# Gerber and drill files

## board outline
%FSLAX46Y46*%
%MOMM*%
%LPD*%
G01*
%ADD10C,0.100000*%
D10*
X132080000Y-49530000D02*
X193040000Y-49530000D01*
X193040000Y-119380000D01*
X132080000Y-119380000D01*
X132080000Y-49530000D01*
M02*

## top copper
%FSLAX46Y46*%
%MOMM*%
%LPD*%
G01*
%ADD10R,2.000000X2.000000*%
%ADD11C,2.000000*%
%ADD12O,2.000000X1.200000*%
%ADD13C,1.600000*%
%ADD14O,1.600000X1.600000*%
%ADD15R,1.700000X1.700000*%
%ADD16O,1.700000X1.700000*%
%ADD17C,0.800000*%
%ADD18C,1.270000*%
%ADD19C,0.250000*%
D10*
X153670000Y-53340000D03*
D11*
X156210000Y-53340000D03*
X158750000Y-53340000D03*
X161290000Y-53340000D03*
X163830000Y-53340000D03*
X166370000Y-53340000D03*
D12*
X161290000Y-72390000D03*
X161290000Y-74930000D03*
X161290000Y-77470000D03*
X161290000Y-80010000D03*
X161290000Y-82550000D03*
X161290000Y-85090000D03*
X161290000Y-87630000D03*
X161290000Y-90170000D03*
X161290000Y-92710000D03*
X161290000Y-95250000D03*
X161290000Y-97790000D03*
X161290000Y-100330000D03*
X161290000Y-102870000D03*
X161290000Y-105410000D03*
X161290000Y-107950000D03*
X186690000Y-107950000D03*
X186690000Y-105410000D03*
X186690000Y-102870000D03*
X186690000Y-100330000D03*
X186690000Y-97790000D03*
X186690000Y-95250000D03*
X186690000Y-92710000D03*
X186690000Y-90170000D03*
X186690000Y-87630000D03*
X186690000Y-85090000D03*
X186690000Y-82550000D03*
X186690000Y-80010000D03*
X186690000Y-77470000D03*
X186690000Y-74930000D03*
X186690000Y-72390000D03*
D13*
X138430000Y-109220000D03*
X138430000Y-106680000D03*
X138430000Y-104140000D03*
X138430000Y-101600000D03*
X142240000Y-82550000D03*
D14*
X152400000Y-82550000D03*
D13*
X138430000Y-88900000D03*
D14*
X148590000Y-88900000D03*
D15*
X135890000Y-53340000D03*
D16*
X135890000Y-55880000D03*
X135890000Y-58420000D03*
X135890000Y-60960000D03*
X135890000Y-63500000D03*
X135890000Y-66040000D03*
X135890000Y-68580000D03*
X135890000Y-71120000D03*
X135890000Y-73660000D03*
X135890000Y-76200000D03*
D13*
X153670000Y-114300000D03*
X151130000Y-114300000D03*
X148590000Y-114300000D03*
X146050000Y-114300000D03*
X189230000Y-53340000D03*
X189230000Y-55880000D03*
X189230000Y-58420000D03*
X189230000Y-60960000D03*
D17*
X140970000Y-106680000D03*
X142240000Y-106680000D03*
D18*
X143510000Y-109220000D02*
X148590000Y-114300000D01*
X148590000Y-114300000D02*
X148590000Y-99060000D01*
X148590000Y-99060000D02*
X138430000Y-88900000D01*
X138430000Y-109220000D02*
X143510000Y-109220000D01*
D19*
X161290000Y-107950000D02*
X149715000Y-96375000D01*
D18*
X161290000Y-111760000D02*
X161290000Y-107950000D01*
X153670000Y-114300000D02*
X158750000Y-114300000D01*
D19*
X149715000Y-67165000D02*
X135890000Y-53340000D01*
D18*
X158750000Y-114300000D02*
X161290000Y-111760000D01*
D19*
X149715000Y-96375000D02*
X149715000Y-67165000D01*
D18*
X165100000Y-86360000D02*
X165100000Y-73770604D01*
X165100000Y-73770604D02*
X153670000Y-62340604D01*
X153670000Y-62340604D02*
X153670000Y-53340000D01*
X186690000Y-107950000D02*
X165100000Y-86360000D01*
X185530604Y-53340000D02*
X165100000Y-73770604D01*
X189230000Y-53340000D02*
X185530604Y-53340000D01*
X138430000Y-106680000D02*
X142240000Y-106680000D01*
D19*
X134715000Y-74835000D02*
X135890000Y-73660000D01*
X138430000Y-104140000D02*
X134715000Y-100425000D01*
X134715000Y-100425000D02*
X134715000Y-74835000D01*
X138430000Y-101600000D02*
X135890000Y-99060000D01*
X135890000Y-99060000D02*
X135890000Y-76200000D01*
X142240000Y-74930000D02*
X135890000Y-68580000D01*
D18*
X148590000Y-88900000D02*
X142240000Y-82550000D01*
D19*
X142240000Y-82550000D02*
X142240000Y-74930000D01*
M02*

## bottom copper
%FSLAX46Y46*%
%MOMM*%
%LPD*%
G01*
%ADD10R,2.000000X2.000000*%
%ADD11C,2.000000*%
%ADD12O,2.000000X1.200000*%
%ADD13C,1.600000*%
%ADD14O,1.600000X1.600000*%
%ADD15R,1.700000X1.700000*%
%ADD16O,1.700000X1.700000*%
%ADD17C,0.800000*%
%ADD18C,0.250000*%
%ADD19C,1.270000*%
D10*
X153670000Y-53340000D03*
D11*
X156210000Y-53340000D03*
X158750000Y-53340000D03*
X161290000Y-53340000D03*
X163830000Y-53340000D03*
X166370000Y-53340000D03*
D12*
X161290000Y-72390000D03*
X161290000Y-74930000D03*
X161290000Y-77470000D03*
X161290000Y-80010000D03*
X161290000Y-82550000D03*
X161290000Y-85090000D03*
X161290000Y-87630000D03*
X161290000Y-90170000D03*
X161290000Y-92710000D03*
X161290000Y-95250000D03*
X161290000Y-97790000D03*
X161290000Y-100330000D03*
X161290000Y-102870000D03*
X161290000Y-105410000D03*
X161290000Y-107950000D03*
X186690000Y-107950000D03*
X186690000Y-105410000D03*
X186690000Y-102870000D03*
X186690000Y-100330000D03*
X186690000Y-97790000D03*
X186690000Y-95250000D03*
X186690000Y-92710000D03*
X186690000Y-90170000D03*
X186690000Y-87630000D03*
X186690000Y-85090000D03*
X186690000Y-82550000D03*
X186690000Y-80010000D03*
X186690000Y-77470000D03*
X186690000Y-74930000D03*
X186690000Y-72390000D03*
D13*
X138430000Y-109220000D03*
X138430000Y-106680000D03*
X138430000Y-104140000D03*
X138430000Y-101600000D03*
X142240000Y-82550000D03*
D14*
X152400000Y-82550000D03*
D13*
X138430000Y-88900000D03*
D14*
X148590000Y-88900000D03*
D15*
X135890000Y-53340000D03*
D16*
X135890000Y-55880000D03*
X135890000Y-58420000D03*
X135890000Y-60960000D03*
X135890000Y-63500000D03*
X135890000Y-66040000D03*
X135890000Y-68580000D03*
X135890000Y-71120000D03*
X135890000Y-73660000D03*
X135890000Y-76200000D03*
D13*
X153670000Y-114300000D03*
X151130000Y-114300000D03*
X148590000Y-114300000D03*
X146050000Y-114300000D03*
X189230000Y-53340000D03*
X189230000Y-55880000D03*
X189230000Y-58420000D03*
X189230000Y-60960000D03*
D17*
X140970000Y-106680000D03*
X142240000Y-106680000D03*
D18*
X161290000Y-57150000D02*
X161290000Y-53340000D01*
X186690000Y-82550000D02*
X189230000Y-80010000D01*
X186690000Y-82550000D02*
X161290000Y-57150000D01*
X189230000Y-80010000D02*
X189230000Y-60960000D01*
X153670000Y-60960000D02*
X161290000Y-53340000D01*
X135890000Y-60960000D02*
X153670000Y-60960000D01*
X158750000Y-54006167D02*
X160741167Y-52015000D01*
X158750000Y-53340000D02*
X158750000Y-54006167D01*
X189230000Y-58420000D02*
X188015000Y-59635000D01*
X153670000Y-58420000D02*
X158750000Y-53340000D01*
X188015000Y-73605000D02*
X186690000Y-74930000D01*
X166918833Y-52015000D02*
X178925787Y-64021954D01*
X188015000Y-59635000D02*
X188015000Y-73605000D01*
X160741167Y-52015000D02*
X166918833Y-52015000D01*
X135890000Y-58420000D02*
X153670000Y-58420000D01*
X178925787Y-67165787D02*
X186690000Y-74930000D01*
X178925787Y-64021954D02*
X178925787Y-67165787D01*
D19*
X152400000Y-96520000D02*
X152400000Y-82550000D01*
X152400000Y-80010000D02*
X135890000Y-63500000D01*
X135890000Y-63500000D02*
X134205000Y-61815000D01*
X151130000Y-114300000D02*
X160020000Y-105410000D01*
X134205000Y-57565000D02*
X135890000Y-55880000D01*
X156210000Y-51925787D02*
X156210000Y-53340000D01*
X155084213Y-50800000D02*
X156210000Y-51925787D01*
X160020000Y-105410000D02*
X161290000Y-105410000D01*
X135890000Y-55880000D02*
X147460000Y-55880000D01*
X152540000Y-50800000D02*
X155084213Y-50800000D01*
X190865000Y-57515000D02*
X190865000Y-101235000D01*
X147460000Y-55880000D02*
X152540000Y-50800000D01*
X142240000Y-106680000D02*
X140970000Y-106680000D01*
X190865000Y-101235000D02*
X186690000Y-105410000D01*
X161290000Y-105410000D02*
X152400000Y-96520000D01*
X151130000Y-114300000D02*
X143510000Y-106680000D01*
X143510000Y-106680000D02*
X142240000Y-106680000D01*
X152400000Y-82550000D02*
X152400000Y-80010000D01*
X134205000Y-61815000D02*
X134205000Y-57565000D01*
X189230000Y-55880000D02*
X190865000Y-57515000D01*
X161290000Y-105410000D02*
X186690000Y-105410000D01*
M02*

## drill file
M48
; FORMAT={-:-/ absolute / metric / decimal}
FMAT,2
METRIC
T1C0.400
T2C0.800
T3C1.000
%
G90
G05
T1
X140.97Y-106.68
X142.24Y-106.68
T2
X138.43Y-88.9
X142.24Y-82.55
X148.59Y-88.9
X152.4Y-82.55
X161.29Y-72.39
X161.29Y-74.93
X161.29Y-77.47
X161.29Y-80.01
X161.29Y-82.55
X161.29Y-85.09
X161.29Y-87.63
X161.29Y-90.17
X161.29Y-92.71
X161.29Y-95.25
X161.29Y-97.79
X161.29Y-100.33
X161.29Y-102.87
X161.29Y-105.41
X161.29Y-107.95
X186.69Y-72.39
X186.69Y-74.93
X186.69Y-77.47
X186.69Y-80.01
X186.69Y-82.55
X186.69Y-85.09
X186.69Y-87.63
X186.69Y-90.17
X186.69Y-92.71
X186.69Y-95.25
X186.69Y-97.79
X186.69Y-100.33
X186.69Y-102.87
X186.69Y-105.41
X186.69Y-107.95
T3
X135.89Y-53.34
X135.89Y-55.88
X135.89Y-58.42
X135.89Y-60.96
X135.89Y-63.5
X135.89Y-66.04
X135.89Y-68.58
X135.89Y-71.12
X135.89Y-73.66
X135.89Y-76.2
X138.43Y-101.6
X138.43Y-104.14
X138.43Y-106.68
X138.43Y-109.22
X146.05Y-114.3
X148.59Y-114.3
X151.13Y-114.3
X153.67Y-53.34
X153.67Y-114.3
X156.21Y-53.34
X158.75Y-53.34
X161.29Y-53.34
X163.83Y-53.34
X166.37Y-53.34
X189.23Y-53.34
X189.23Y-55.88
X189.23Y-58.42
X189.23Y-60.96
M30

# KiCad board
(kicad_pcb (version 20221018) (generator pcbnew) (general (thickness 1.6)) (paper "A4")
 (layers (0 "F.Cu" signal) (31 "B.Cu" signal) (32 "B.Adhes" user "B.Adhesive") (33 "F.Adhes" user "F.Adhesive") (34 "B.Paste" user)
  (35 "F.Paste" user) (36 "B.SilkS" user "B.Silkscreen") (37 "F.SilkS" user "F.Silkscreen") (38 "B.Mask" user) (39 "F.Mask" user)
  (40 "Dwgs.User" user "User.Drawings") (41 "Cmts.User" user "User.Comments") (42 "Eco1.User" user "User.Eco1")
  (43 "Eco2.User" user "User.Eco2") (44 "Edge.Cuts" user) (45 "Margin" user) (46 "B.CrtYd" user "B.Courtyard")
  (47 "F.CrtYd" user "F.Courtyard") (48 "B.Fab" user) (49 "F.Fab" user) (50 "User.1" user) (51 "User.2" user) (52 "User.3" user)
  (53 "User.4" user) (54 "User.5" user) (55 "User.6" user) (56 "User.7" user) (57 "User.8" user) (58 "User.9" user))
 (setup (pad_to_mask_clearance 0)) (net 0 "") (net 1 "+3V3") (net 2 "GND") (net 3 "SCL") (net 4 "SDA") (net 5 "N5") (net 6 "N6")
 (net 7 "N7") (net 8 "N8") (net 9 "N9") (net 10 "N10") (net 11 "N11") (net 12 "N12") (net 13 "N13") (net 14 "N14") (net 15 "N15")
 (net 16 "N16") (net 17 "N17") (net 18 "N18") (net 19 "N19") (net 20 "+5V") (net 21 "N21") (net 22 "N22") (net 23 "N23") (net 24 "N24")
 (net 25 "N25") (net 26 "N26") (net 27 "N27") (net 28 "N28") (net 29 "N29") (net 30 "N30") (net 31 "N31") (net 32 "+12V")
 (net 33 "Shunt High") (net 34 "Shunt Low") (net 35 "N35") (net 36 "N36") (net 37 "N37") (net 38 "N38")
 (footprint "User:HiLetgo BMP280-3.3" (layer "F.Cu") (at 153.67 53.34 90)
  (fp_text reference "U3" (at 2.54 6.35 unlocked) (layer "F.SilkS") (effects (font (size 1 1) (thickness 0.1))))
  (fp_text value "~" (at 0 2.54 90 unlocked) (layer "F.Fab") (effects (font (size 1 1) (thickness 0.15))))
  (pad "1" thru_hole rect (at 0 0 90) (size 2 2) (drill 1) (layers "*.Cu" "*.Mask") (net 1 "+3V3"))
  (pad "2" thru_hole circle (at 0 2.54 90) (size 2 2) (drill 1) (layers "*.Cu" "*.Mask") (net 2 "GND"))
  (pad "3" thru_hole circle (at 0 5.08 90) (size 2 2) (drill 1) (layers "*.Cu" "*.Mask") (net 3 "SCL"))
  (pad "4" thru_hole circle (at 0 7.62 90) (size 2 2) (drill 1) (layers "*.Cu" "*.Mask") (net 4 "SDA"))
  (pad "5" thru_hole circle (at 0 10.16 90) (size 2 2) (drill 1) (layers "*.Cu" "*.Mask") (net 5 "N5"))
  (pad "6" thru_hole circle (at 0 12.7 90) (size 2 2) (drill 1) (layers "*.Cu" "*.Mask") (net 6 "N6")))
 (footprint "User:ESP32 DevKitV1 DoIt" (layer "F.Cu") (at 158.75 69.85)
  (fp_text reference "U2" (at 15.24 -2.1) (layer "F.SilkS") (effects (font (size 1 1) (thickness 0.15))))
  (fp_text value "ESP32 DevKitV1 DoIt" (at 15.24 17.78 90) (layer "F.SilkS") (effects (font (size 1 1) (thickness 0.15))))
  (pad "1" thru_hole oval (at 2.54 2.54 270) (size 1.2 2) (drill 0.8) (layers "*.Cu" "*.Mask") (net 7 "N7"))
  (pad "2" thru_hole oval (at 2.54 5.08 270) (size 1.2 2) (drill 0.8) (layers "*.Cu" "*.Mask") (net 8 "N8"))
  (pad "3" thru_hole oval (at 2.54 7.62 270) (size 1.2 2) (drill 0.8) (layers "*.Cu" "*.Mask") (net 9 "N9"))
  (pad "4" thru_hole oval (at 2.54 10.16 270) (size 1.2 2) (drill 0.8) (layers "*.Cu" "*.Mask") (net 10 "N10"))
  (pad "5" thru_hole oval (at 2.54 12.7 270) (size 1.2 2) (drill 0.8) (layers "*.Cu" "*.Mask") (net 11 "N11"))
  (pad "6" thru_hole oval (at 2.54 15.24 270) (size 1.2 2) (drill 0.8) (layers "*.Cu" "*.Mask") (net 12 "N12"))
  (pad "7" thru_hole oval (at 2.54 17.78 270) (size 1.2 2) (drill 0.8) (layers "*.Cu" "*.Mask") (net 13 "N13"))
  (pad "8" thru_hole oval (at 2.54 20.32 270) (size 1.2 2) (drill 0.8) (layers "*.Cu" "*.Mask") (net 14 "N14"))
  (pad "9" thru_hole oval (at 2.54 22.86 270) (size 1.2 2) (drill 0.8) (layers "*.Cu" "*.Mask") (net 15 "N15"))
  (pad "10" thru_hole oval (at 2.54 25.4 270) (size 1.2 2) (drill 0.8) (layers "*.Cu" "*.Mask") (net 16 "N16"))
  (pad "11" thru_hole oval (at 2.54 27.94 270) (size 1.2 2) (drill 0.8) (layers "*.Cu" "*.Mask") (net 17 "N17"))
  (pad "12" thru_hole oval (at 2.54 30.48 270) (size 1.2 2) (drill 0.8) (layers "*.Cu" "*.Mask") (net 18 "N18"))
  (pad "13" thru_hole oval (at 2.54 33.02 270) (size 1.2 2) (drill 0.8) (layers "*.Cu" "*.Mask") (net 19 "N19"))
  (pad "14" thru_hole oval (at 2.54 35.56 270) (size 1.2 2) (drill 0.8) (layers "*.Cu" "*.Mask") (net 2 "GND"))
  (pad "15" thru_hole oval (at 2.54 38.1 270) (size 1.2 2) (drill 0.8) (layers "*.Cu" "*.Mask") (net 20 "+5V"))
  (pad "16" thru_hole oval (at 27.94 38.1 270) (size 1.2 2) (drill 0.8) (layers "*.Cu" "*.Mask") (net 1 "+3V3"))
  (pad "17" thru_hole oval (at 27.94 35.56 270) (size 1.2 2) (drill 0.8) (layers "*.Cu" "*.Mask") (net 2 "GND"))
  (pad "18" thru_hole oval (at 27.94 33.02 270) (size 1.2 2) (drill 0.8) (layers "*.Cu" "*.Mask") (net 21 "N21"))
  (pad "19" thru_hole oval (at 27.94 30.48 270) (size 1.2 2) (drill 0.8) (layers "*.Cu" "*.Mask") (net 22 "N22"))
  (pad "20" thru_hole oval (at 27.94 27.94 270) (size 1.2 2) (drill 0.8) (layers "*.Cu" "*.Mask") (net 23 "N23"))
  (pad "21" thru_hole oval (at 27.94 25.4 270) (size 1.2 2) (drill 0.8) (layers "*.Cu" "*.Mask") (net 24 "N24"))
  (pad "22" thru_hole oval (at 27.94 22.86 270) (size 1.2 2) (drill 0.8) (layers "*.Cu" "*.Mask") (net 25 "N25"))
  (pad "23" thru_hole oval (at 27.94 20.32 270) (size 1.2 2) (drill 0.8) (layers "*.Cu" "*.Mask") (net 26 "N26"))
  (pad "24" thru_hole oval (at 27.94 17.78 270) (size 1.2 2) (drill 0.8) (layers "*.Cu" "*.Mask") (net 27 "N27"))
  (pad "25" thru_hole oval (at 27.94 15.24 270) (size 1.2 2) (drill 0.8) (layers "*.Cu" "*.Mask") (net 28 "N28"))
  (pad "26" thru_hole oval (at 27.94 12.7 270) (size 1.2 2) (drill 0.8) (layers "*.Cu" "*.Mask") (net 4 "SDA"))
  (pad "27" thru_hole oval (at 27.94 10.16 270) (size 1.2 2) (drill 0.8) (layers "*.Cu" "*.Mask") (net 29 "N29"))
  (pad "28" thru_hole oval (at 27.94 7.62 270) (size 1.2 2) (drill 0.8) (layers "*.Cu" "*.Mask") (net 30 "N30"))
  (pad "29" thru_hole oval (at 27.94 5.08 270) (size 1.2 2) (drill 0.8) (layers "*.Cu" "*.Mask") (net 3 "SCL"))
  (pad "30" thru_hole oval (at 27.94 2.54 270) (size 1.2 2) (drill 0.8) (layers "*.Cu" "*.Mask") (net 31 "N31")))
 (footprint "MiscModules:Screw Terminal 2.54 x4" (layer "F.Cu") (at 140.97 96.52 180)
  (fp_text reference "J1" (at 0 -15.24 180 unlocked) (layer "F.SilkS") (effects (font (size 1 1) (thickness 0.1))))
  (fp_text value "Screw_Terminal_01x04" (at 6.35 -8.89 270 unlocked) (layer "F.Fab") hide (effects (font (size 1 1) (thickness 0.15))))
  (pad "1" thru_hole circle (at 2.54 -12.7 90) (size 1.6 1.6) (drill 1) (layers "*.Cu" "*.Mask") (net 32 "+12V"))
  (pad "2" thru_hole circle (at 2.54 -10.16 90) (size 1.6 1.6) (drill 1) (layers "*.Cu" "*.Mask") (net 2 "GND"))
  (pad "3" thru_hole circle (at 2.54 -7.62 90) (size 1.6 1.6) (drill 1) (layers "*.Cu" "*.Mask") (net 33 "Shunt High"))
  (pad "4" thru_hole circle (at 2.54 -5.08 90) (size 1.6 1.6) (drill 1) (layers "*.Cu" "*.Mask") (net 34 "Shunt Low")))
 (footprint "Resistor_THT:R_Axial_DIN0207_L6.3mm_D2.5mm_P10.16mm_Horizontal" (layer "F.Cu") (at 142.24 82.55)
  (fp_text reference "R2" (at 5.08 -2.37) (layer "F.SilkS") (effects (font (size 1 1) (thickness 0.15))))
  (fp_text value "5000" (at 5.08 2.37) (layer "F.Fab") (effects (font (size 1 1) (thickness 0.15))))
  (pad "1" thru_hole circle (at 0 0) (size 1.6 1.6) (drill 0.8) (layers "*.Cu" "*.Mask") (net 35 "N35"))
  (pad "2" thru_hole oval (at 10.16 0) (size 1.6 1.6) (drill 0.8) (layers "*.Cu" "*.Mask") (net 2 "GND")))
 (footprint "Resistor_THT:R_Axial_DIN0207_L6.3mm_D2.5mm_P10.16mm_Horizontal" (layer "F.Cu") (at 138.43 88.9)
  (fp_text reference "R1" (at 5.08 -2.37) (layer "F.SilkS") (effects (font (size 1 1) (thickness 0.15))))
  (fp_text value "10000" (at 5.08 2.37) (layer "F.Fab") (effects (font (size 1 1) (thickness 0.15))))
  (pad "1" thru_hole circle (at 0 0) (size 1.6 1.6) (drill 0.8) (layers "*.Cu" "*.Mask") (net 32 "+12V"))
  (pad "2" thru_hole oval (at 10.16 0) (size 1.6 1.6) (drill 0.8) (layers "*.Cu" "*.Mask") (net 35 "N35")))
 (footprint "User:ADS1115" (layer "F.Cu") (at 135.89 53.34)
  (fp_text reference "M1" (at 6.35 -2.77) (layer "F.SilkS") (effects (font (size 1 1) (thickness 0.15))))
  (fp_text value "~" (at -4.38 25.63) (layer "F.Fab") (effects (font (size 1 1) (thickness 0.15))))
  (pad "1" thru_hole rect (at 0 0) (size 1.7 1.7) (drill 1) (layers "*.Cu" "*.Mask") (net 20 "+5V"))
  (pad "2" thru_hole oval (at 0 2.54) (size 1.7 1.7) (drill 1) (layers "*.Cu" "*.Mask") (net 2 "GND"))
  (pad "3" thru_hole oval (at 0 5.08) (size 1.7 1.7) (drill 1) (layers "*.Cu" "*.Mask") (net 3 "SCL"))
  (pad "4" thru_hole oval (at 0 7.62) (size 1.7 1.7) (drill 1) (layers "*.Cu" "*.Mask") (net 4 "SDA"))
  (pad "5" thru_hole oval (at 0 10.16) (size 1.7 1.7) (drill 1) (layers "*.Cu" "*.Mask") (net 2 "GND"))
  (pad "6" thru_hole oval (at 0 12.7) (size 1.7 1.7) (drill 1) (layers "*.Cu" "*.Mask") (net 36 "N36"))
  (pad "7" thru_hole oval (at 0 15.24) (size 1.7 1.7) (drill 1) (layers "*.Cu" "*.Mask") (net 35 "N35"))
  (pad "8" thru_hole oval (at 0 17.78) (size 1.7 1.7) (drill 1) (layers "*.Cu" "*.Mask") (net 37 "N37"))
  (pad "9" thru_hole oval (at 0 20.32) (size 1.7 1.7) (drill 1) (layers "*.Cu" "*.Mask") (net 33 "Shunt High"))
  (pad "10" thru_hole oval (at 0 22.86) (size 1.7 1.7) (drill 1) (layers "*.Cu" "*.Mask") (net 34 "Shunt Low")))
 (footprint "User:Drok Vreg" (layer "F.Cu") (at 149.86 111.76 -90)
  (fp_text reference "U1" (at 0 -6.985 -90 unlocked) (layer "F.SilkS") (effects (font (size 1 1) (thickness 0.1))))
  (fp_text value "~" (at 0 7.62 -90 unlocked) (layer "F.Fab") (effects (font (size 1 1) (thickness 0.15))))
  (pad "1" thru_hole circle (at 2.54 -3.81 180) (size 1.6 1.6) (drill 1) (layers "*.Cu" "*.Mask") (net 20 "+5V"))
  (pad "2" thru_hole circle (at 2.54 -1.27 180) (size 1.6 1.6) (drill 1) (layers "*.Cu" "*.Mask") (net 2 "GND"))
  (pad "3" thru_hole circle (at 2.54 1.27 180) (size 1.6 1.6) (drill 1) (layers "*.Cu" "*.Mask") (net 32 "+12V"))
  (pad "4" thru_hole circle (at 2.54 3.81 180) (size 1.6 1.6) (drill 1) (layers "*.Cu" "*.Mask") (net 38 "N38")))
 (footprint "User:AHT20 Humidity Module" (layer "F.Cu") (at 186.69 57.15)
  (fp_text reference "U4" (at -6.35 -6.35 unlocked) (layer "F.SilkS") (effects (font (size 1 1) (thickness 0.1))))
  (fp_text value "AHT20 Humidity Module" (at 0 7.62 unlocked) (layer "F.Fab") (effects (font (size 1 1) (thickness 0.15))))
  (pad "1" thru_hole circle (at 2.54 -3.81 270) (size 1.6 1.6) (drill 1) (layers "*.Cu" "*.Mask") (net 1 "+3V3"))
  (pad "2" thru_hole circle (at 2.54 -1.27 270) (size 1.6 1.6) (drill 1) (layers "*.Cu" "*.Mask") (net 2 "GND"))
  (pad "3" thru_hole circle (at 2.54 1.27 270) (size 1.6 1.6) (drill 1) (layers "*.Cu" "*.Mask") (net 3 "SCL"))
  (pad "4" thru_hole circle (at 2.54 3.81 270) (size 1.6 1.6) (drill 1) (layers "*.Cu" "*.Mask") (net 4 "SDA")))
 (gr_rect (start 132.08 49.53) (end 193.04 119.38) (stroke (width 0.1) (type default)) (fill none) (layer "Edge.Cuts"))
 (segment (start 143.51 109.22) (end 148.59 114.3) (width 1.27) (layer "F.Cu") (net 32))
 (segment (start 148.59 114.3) (end 148.59 99.06) (width 1.27) (layer "F.Cu") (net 32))
 (segment (start 148.59 99.06) (end 138.43 88.9) (width 1.27) (layer "F.Cu") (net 32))
 (segment (start 138.43 109.22) (end 143.51 109.22) (width 1.27) (layer "F.Cu") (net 32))
 (segment (start 161.29 107.95) (end 149.715 96.375) (width 0.25) (layer "F.Cu") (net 20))
 (segment (start 161.29 111.76) (end 161.29 107.95) (width 1.27) (layer "F.Cu") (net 20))
 (segment (start 153.67 114.3) (end 158.75 114.3) (width 1.27) (layer "F.Cu") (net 20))
 (segment (start 149.715 67.165) (end 135.89 53.34) (width 0.25) (layer "F.Cu") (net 20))
 (segment (start 158.75 114.3) (end 161.29 111.76) (width 1.27) (layer "F.Cu") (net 20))
 (segment (start 149.715 96.375) (end 149.715 67.165) (width 0.25) (layer "F.Cu") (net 20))
 (segment (start 165.1 86.36) (end 165.1 73.770604) (width 1.27) (layer "F.Cu") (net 1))
 (segment (start 165.1 73.770604) (end 153.67 62.340604) (width 1.27) (layer "F.Cu") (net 1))
 (segment (start 153.67 62.340604) (end 153.67 53.34) (width 1.27) (layer "F.Cu") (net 1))
 (segment (start 186.69 107.95) (end 165.1 86.36) (width 1.27) (layer "F.Cu") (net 1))
 (segment (start 185.530604 53.34) (end 165.1 73.770604) (width 1.27) (layer "F.Cu") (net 1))
 (segment (start 189.23 53.34) (end 185.530604 53.34) (width 1.27) (layer "F.Cu") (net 1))
 (segment (start 161.29 57.15) (end 161.29 53.34) (width 0.25) (layer "B.Cu") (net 4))
 (segment (start 186.69 82.55) (end 189.23 80.01) (width 0.25) (layer "B.Cu") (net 4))
 (segment (start 186.69 82.55) (end 161.29 57.15) (width 0.25) (layer "B.Cu") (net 4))
 (segment (start 189.23 80.01) (end 189.23 60.96) (width 0.25) (layer "B.Cu") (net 4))
 (segment (start 153.67 60.96) (end 161.29 53.34) (width 0.25) (layer "B.Cu") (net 4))
 (segment (start 135.89 60.96) (end 153.67 60.96) (width 0.25) (layer "B.Cu") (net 4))
 (segment (start 158.75 54.006167) (end 160.741167 52.015) (width 0.25) (layer "B.Cu") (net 3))
 (segment (start 158.75 53.34) (end 158.75 54.006167) (width 0.25) (layer "B.Cu") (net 3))
 (segment (start 189.23 58.42) (end 188.015 59.635) (width 0.25) (layer "B.Cu") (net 3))
 (segment (start 153.67 58.42) (end 158.75 53.34) (width 0.25) (layer "B.Cu") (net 3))
 (segment (start 188.015 73.605) (end 186.69 74.93) (width 0.25) (layer "B.Cu") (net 3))
 (segment (start 166.918833 52.015) (end 178.925787 64.021954) (width 0.25) (layer "B.Cu") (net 3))
 (segment (start 188.015 59.635) (end 188.015 73.605) (width 0.25) (layer "B.Cu") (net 3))
 (segment (start 160.741167 52.015) (end 166.918833 52.015) (width 0.25) (layer "B.Cu") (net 3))
 (segment (start 135.89 58.42) (end 153.67 58.42) (width 0.25) (layer "B.Cu") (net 3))
 (segment (start 178.925787 67.165787) (end 186.69 74.93) (width 0.25) (layer "B.Cu") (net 3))
 (segment (start 178.925787 64.021954) (end 178.925787 67.165787) (width 0.25) (layer "B.Cu") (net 3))
 (segment (start 138.43 106.68) (end 142.24 106.68) (width 1.27) (layer "F.Cu") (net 2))
 (via (at 140.97 106.68) (size 0.8) (drill 0.4) (layers "F.Cu" "B.Cu") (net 2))
 (via (at 142.24 106.68) (size 0.8) (drill 0.4) (layers "F.Cu" "B.Cu") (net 2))
 (segment (start 152.4 96.52) (end 152.4 82.55) (width 1.27) (layer "B.Cu") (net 2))
 (segment (start 152.4 80.01) (end 135.89 63.5) (width 1.27) (layer "B.Cu") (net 2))
 (segment (start 135.89 63.5) (end 134.205 61.815) (width 1.27) (layer "B.Cu") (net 2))
 (segment (start 151.13 114.3) (end 160.02 105.41) (width 1.27) (layer "B.Cu") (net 2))
 (segment (start 134.205 57.565) (end 135.89 55.88) (width 1.27) (layer "B.Cu") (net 2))
 (segment (start 156.21 51.925787) (end 156.21 53.34) (width 1.27) (layer "B.Cu") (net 2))
 (segment (start 155.084213 50.8) (end 156.21 51.925787) (width 1.27) (layer "B.Cu") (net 2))
 (segment (start 160.02 105.41) (end 161.29 105.41) (width 1.27) (layer "B.Cu") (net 2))
 (segment (start 135.89 55.88) (end 147.46 55.88) (width 1.27) (layer "B.Cu") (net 2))
 (segment (start 152.54 50.8) (end 155.084213 50.8) (width 1.27) (layer "B.Cu") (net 2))
 (segment (start 190.865 57.515) (end 190.865 101.235) (width 1.27) (layer "B.Cu") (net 2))
 (segment (start 147.46 55.88) (end 152.54 50.8) (width 1.27) (layer "B.Cu") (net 2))
 (segment (start 142.24 106.68) (end 140.97 106.68) (width 1.27) (layer "B.Cu") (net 2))
 (segment (start 190.865 101.235) (end 186.69 105.41) (width 1.27) (layer "B.Cu") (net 2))
 (segment (start 161.29 105.41) (end 152.4 96.52) (width 1.27) (layer "B.Cu") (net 2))
 (segment (start 151.13 114.3) (end 143.51 106.68) (width 1.27) (layer "B.Cu") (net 2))
 (segment (start 143.51 106.68) (end 142.24 106.68) (width 1.27) (layer "B.Cu") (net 2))
 (segment (start 152.4 82.55) (end 152.4 80.01) (width 1.27) (layer "B.Cu") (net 2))
 (segment (start 134.205 61.815) (end 134.205 57.565) (width 1.27) (layer "B.Cu") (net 2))
 (segment (start 189.23 55.88) (end 190.865 57.515) (width 1.27) (layer "B.Cu") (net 2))
 (segment (start 161.29 105.41) (end 186.69 105.41) (width 1.27) (layer "B.Cu") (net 2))
 (segment (start 134.715 74.835) (end 135.89 73.66) (width 0.25) (layer "F.Cu") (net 33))
 (segment (start 138.43 104.14) (end 134.715 100.425) (width 0.25) (layer "F.Cu") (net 33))
 (segment (start 134.715 100.425) (end 134.715 74.835) (width 0.25) (layer "F.Cu") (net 33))
 (segment (start 138.43 101.6) (end 135.89 99.06) (width 0.25) (layer "F.Cu") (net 34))
 (segment (start 135.89 99.06) (end 135.89 76.2) (width 0.25) (layer "F.Cu") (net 34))
 (segment (start 142.24 74.93) (end 135.89 68.58) (width 0.25) (layer "F.Cu") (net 35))
 (segment (start 148.59 88.9) (end 142.24 82.55) (width 1.27) (layer "F.Cu") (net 35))
 (segment (start 142.24 82.55) (end 142.24 74.93) (width 0.25) (layer "F.Cu") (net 35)))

